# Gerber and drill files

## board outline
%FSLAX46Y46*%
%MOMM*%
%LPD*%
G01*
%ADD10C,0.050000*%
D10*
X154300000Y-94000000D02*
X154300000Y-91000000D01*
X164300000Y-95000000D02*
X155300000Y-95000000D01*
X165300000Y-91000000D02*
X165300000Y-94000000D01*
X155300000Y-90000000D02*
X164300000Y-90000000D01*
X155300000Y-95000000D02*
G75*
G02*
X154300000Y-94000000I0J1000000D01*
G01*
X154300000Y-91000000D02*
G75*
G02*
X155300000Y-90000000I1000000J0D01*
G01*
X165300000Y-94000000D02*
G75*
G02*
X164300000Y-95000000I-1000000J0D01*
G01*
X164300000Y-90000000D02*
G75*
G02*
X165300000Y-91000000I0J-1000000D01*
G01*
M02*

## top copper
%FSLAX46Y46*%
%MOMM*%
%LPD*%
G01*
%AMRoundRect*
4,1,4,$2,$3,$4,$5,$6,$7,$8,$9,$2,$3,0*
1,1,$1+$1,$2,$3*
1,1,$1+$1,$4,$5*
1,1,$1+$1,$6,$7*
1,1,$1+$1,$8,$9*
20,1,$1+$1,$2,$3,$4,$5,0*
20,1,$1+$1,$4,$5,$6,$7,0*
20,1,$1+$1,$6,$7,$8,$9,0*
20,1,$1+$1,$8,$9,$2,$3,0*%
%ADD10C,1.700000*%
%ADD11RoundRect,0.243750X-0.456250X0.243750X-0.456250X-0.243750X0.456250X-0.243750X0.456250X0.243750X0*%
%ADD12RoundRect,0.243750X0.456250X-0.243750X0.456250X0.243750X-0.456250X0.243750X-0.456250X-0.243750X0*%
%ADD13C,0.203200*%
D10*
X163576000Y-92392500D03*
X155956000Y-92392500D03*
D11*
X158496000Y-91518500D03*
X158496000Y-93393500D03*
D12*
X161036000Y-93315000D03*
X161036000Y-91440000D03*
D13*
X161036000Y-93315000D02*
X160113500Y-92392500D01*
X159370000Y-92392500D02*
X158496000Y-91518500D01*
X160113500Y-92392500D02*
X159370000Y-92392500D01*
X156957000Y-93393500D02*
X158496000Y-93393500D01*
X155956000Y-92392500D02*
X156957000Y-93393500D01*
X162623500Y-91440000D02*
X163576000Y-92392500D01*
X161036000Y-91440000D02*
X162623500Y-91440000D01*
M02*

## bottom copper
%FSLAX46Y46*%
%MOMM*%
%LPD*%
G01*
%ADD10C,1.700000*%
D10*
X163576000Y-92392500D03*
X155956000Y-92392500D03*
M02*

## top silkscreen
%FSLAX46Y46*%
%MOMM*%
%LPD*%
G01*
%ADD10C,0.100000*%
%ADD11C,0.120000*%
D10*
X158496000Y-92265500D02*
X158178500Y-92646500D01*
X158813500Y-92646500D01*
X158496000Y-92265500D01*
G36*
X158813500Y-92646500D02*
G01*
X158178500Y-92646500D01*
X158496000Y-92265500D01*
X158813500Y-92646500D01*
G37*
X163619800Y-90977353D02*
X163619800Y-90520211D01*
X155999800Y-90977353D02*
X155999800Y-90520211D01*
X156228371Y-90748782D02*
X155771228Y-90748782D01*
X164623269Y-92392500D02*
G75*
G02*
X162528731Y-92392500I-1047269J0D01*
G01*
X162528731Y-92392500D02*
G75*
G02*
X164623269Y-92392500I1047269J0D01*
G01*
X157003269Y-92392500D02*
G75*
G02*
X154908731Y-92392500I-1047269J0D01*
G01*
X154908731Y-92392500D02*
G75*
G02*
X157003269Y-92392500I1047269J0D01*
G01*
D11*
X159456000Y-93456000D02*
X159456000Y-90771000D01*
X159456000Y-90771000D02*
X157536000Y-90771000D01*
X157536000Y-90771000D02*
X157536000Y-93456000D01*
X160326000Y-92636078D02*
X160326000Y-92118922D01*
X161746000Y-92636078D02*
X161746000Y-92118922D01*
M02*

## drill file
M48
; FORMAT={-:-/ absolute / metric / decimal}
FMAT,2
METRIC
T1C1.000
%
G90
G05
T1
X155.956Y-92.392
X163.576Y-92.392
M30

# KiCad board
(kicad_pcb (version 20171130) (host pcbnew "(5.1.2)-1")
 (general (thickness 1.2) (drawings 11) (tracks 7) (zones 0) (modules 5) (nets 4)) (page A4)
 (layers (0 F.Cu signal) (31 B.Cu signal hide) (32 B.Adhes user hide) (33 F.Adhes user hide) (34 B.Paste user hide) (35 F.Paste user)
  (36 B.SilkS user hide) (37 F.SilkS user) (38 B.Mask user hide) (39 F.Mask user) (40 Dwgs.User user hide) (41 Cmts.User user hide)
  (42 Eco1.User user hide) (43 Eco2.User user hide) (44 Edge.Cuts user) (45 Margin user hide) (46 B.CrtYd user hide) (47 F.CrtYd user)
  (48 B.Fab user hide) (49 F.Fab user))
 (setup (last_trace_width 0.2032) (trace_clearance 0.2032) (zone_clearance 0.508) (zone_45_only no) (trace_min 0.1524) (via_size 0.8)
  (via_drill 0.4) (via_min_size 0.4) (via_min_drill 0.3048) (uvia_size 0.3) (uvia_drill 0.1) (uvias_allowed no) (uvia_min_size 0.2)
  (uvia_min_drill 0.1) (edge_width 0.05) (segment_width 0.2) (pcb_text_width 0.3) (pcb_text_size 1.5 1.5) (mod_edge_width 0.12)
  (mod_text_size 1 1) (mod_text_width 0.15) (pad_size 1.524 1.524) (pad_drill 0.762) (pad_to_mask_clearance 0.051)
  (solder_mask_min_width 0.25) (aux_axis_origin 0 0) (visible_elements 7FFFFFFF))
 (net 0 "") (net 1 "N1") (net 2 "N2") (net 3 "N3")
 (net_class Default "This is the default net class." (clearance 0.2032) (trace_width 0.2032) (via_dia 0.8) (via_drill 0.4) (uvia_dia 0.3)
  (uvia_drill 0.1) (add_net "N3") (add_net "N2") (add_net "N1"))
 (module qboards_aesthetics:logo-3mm (layer B.Cu) (at 160 91.9 180)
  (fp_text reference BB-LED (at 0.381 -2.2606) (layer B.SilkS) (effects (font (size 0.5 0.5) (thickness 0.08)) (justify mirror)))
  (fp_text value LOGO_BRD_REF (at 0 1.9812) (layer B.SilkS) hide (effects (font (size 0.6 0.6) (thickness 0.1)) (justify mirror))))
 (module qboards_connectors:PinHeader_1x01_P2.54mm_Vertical (layer F.Cu) (at 163.576 92.3925 90)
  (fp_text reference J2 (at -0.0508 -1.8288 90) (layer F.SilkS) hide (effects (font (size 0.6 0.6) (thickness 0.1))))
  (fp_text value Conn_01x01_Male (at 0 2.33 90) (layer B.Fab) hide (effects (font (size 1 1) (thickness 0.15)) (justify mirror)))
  (fp_circle (center 0 0) (end 0.8128 0.6604) (layer F.SilkS) (width 0.1))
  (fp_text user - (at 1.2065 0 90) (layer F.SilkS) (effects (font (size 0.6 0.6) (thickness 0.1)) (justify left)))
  (pad 1 thru_hole circle (at 0 0 90) (size 1.7 1.7) (drill 1) (layers *.Cu *.Mask) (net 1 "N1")))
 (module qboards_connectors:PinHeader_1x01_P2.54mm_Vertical (layer F.Cu) (at 155.956 92.3925 90)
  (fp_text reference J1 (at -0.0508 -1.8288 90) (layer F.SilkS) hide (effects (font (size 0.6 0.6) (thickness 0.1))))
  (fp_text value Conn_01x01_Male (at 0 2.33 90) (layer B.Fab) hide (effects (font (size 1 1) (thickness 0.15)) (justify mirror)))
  (fp_circle (center 0 0) (end 0.8128 0.6604) (layer F.SilkS) (width 0.1))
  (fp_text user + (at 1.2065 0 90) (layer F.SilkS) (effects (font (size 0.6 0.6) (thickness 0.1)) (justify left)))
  (pad 1 thru_hole circle (at 0 0 90) (size 1.7 1.7) (drill 1) (layers *.Cu *.Mask) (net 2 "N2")))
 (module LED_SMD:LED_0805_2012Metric (layer F.Cu) (at 158.496 92.456 270)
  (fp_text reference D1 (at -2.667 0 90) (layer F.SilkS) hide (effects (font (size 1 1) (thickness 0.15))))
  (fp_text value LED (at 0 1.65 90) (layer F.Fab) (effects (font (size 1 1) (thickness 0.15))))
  (fp_line (start 1 -0.96) (end -1.685 -0.96) (layer F.SilkS) (width 0.12))
  (fp_line (start -1.685 -0.96) (end -1.685 0.96) (layer F.SilkS) (width 0.12))
  (fp_line (start -1.685 0.96) (end 1 0.96) (layer F.SilkS) (width 0.12))
  (pad 1 smd roundrect (at -0.9375 0 270) (size 0.975 1.4) (layers F.Cu F.Paste F.Mask) (roundrect_rratio 0.25) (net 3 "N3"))
  (pad 2 smd roundrect (at 0.9375 0 270) (size 0.975 1.4) (layers F.Cu F.Paste F.Mask) (roundrect_rratio 0.25) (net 2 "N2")))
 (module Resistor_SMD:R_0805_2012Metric (layer F.Cu) (at 161.036 92.3775 90)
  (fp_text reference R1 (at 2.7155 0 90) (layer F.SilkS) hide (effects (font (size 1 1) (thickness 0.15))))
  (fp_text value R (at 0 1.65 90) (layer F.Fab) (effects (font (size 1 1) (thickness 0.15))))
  (fp_line (start -0.258578 -0.71) (end 0.258578 -0.71) (layer F.SilkS) (width 0.12))
  (fp_line (start -0.258578 0.71) (end 0.258578 0.71) (layer F.SilkS) (width 0.12))
  (pad 1 smd roundrect (at -0.9375 0 90) (size 0.975 1.4) (layers F.Cu F.Paste F.Mask) (roundrect_rratio 0.25) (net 3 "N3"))
  (pad 2 smd roundrect (at 0.9375 0 90) (size 0.975 1.4) (layers F.Cu F.Paste F.Mask) (roundrect_rratio 0.25) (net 1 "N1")))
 (gr_line (start 154.3 94) (end 154.3 91) (layer Edge.Cuts) (width 0.05))
 (gr_line (start 164.3 95) (end 155.3 95) (layer Edge.Cuts) (width 0.05))
 (gr_line (start 165.3 91) (end 165.3 94) (layer Edge.Cuts) (width 0.05))
 (gr_line (start 155.3 90) (end 164.3 90) (layer Edge.Cuts) (width 0.05))
 (gr_arc (start 155.3 94) (end 154.3 94) (angle -90) (layer Edge.Cuts) (width 0.05))
 (gr_arc (start 155.3 91) (end 155.3 90) (angle -90) (layer Edge.Cuts) (width 0.05))
 (gr_arc (start 164.3 94) (end 164.3 95) (angle -90) (layer Edge.Cuts) (width 0.05))
 (gr_arc (start 164.3 91) (end 165.3 91) (angle -90) (layer Edge.Cuts) (width 0.05))
 (gr_poly (pts (xy 158.496 92.2655) (xy 158.1785 92.6465) (xy 158.8135 92.6465)) (layer F.SilkS) (width 0.1))
 (segment (start 161.036 93.315) (end 160.1135 92.3925) (width 0.2032) (layer F.Cu) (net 3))
 (segment (start 159.37 92.3925) (end 158.496 91.5185) (width 0.2032) (layer F.Cu) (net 3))
 (segment (start 160.1135 92.3925) (end 159.37 92.3925) (width 0.2032) (layer F.Cu) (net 3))
 (segment (start 156.957 93.3935) (end 158.496 93.3935) (width 0.2032) (layer F.Cu) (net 2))
 (segment (start 155.956 92.3925) (end 156.957 93.3935) (width 0.2032) (layer F.Cu) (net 2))
 (segment (start 162.6235 91.44) (end 163.576 92.3925) (width 0.2032) (layer F.Cu) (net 1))
 (segment (start 161.036 91.44) (end 162.6235 91.44) (width 0.2032) (layer F.Cu) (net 1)))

